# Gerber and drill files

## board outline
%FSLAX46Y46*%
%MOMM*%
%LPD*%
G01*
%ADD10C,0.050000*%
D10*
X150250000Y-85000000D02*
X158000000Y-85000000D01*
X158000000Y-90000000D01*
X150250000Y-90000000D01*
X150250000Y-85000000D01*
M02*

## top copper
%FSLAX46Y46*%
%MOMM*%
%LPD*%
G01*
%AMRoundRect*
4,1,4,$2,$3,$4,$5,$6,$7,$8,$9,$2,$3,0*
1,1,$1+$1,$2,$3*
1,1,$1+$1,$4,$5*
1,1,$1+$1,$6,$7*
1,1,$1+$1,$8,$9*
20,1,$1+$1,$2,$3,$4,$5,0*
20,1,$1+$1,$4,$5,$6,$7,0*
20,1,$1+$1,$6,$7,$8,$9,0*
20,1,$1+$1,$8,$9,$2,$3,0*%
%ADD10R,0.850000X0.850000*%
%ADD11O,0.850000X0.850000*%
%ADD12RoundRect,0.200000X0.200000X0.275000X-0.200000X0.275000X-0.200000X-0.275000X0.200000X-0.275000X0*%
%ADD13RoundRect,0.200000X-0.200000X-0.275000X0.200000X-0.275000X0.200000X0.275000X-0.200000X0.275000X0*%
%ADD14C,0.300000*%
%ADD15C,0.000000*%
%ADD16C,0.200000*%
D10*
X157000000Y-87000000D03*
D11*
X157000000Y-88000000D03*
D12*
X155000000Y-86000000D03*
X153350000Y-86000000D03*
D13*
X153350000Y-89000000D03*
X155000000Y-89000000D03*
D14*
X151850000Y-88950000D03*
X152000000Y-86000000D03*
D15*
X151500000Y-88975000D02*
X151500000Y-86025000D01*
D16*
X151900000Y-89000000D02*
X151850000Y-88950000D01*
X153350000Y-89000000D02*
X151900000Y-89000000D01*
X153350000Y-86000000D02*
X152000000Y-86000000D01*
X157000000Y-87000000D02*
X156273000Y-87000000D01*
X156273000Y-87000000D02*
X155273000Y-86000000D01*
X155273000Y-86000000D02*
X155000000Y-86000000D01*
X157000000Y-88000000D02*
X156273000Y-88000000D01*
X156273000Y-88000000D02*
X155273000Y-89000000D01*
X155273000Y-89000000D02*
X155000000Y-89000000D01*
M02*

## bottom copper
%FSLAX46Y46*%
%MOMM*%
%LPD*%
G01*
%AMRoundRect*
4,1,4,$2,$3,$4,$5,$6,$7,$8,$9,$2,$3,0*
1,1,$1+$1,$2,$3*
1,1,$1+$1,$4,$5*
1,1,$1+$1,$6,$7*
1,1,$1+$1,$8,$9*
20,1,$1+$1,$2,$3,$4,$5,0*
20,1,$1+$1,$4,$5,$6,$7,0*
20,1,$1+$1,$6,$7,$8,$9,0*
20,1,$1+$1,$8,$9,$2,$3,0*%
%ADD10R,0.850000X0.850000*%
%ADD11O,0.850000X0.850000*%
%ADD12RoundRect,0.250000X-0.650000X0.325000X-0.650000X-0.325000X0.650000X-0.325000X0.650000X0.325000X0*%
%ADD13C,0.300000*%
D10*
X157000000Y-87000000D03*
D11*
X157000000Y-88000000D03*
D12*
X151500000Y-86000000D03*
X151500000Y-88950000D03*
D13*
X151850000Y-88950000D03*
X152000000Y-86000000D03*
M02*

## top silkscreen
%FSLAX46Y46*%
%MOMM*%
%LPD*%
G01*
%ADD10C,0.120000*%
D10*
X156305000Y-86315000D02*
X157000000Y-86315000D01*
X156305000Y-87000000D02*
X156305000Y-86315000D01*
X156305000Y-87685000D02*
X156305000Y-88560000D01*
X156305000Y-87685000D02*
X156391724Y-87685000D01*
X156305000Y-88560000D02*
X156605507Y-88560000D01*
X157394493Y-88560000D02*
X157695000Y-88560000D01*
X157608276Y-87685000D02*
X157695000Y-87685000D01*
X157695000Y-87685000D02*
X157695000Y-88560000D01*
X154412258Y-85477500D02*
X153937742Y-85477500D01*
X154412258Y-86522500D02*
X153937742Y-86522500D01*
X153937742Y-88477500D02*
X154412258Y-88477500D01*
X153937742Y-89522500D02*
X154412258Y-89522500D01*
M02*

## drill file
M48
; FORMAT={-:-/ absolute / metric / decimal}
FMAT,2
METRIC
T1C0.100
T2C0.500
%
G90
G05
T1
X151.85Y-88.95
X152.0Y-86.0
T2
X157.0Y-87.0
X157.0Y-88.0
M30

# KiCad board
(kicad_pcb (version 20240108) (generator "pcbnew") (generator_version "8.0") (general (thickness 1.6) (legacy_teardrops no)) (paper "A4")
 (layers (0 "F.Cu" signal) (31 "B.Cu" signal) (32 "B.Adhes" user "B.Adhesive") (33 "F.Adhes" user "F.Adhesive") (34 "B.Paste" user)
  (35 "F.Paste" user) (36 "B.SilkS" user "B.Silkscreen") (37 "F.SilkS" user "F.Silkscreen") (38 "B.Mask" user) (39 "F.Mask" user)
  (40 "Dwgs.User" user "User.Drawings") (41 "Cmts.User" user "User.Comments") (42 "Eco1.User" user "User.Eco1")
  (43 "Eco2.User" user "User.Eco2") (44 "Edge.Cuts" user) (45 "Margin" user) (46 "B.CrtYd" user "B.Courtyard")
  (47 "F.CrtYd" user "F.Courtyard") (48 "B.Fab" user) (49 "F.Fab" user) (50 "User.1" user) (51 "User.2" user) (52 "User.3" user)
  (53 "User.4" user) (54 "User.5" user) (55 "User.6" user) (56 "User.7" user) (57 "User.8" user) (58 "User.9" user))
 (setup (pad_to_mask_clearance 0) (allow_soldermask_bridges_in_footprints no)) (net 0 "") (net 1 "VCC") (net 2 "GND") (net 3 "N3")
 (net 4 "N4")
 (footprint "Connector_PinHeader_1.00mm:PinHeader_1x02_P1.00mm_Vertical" (layer "F.Cu") (at 157 87)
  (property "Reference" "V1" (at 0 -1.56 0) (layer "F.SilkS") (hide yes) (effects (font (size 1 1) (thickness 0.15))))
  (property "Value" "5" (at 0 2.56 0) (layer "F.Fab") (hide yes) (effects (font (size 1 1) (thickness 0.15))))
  (fp_line (start -0.695 -0.685) (end 0 -0.685) (stroke (width 0.12) (type solid)) (layer "F.SilkS"))
  (fp_line (start -0.695 0) (end -0.695 -0.685) (stroke (width 0.12) (type solid)) (layer "F.SilkS"))
  (fp_line (start -0.695 0.685) (end -0.695 1.56) (stroke (width 0.12) (type solid)) (layer "F.SilkS"))
  (fp_line (start -0.695 0.685) (end -0.608276 0.685) (stroke (width 0.12) (type solid)) (layer "F.SilkS"))
  (fp_line (start -0.695 1.56) (end -0.394493 1.56) (stroke (width 0.12) (type solid)) (layer "F.SilkS"))
  (fp_line (start 0.394493 1.56) (end 0.695 1.56) (stroke (width 0.12) (type solid)) (layer "F.SilkS"))
  (fp_line (start 0.608276 0.685) (end 0.695 0.685) (stroke (width 0.12) (type solid)) (layer "F.SilkS"))
  (fp_line (start 0.695 0.685) (end 0.695 1.56) (stroke (width 0.12) (type solid)) (layer "F.SilkS"))
  (pad "1" thru_hole rect (at 0 0) (size 0.85 0.85) (drill 0.5) (layers "*.Cu" "*.Mask") (remove_unused_layers no) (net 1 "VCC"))
  (pad "2" thru_hole oval (at 0 1) (size 0.85 0.85) (drill 0.5) (layers "*.Cu" "*.Mask") (remove_unused_layers no) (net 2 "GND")))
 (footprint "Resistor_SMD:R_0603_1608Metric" (layer "F.Cu") (at 154.175 86 180)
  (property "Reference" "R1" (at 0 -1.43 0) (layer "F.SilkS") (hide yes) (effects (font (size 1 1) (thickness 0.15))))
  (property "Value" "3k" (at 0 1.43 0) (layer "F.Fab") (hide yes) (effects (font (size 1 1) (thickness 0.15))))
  (fp_line (start -0.237258 0.5225) (end 0.237258 0.5225) (stroke (width 0.12) (type solid)) (layer "F.SilkS"))
  (fp_line (start -0.237258 -0.5225) (end 0.237258 -0.5225) (stroke (width 0.12) (type solid)) (layer "F.SilkS"))
  (pad "1" smd roundrect (at -0.825 0 180) (size 0.8 0.95) (layers "F.Cu" "F.Paste" "F.Mask") (roundrect_rratio 0.25) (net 1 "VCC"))
  (pad "2" smd roundrect (at 0.825 0 180) (size 0.8 0.95) (layers "F.Cu" "F.Paste" "F.Mask") (roundrect_rratio 0.25) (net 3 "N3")))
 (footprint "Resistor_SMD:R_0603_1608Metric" (layer "F.Cu") (at 154.175 89)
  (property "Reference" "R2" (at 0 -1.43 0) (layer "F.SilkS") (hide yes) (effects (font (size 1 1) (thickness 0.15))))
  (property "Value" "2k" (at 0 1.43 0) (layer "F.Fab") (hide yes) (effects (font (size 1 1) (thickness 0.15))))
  (fp_line (start -0.237258 -0.5225) (end 0.237258 -0.5225) (stroke (width 0.12) (type solid)) (layer "F.SilkS"))
  (fp_line (start -0.237258 0.5225) (end 0.237258 0.5225) (stroke (width 0.12) (type solid)) (layer "F.SilkS"))
  (pad "1" smd roundrect (at -0.825 0) (size 0.8 0.95) (layers "F.Cu" "F.Paste" "F.Mask") (roundrect_rratio 0.25) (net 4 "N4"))
  (pad "2" smd roundrect (at 0.825 0) (size 0.8 0.95) (layers "F.Cu" "F.Paste" "F.Mask") (roundrect_rratio 0.25) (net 2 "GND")))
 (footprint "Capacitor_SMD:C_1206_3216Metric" (layer "B.Cu") (at 151.5 87.475 -90)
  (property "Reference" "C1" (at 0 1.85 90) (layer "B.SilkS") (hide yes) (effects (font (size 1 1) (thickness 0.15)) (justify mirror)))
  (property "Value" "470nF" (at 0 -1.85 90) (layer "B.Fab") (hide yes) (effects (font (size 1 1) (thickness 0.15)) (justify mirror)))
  (pad "1" smd roundrect (at -1.475 0 270) (size 1.15 1.8) (layers "B.Cu" "B.Paste" "B.Mask") (roundrect_rratio 0.217391) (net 3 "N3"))
  (pad "2" smd roundrect (at 1.475 0 270) (size 1.15 1.8) (layers "B.Cu" "B.Paste" "B.Mask") (roundrect_rratio 0.217391) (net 4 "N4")))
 (gr_rect (start 150.25 85) (end 158 90) (stroke (width 0.05) (type default)) (fill none) (layer "Edge.Cuts"))
 (segment (start 151.5 88.975) (end 151.5 86.025) (width 0) (layer "F.Cu") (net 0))
 (segment (start 151.9 89) (end 151.85 88.95) (width 0.2) (layer "F.Cu") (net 4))
 (segment (start 153.35 89) (end 151.9 89) (width 0.2) (layer "F.Cu") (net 4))
 (via micro (at 151.85 88.95) (size 0.3) (drill 0.1) (layers "F.Cu" "B.Cu") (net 4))
 (segment (start 153.35 86) (end 152 86) (width 0.2) (layer "F.Cu") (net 3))
 (via micro (at 152 86) (size 0.3) (drill 0.1) (layers "F.Cu" "B.Cu") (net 3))
 (segment (start 157 87) (end 156.273 87) (width 0.2) (layer "F.Cu") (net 1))
 (segment (start 156.273 87) (end 155.273 86) (width 0.2) (layer "F.Cu") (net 1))
 (segment (start 155.273 86) (end 155 86) (width 0.2) (layer "F.Cu") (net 1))
 (segment (start 157 88) (end 156.273 88) (width 0.2) (layer "F.Cu") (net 2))
 (segment (start 156.273 88) (end 155.273 89) (width 0.2) (layer "F.Cu") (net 2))
 (segment (start 155.273 89) (end 155 89) (width 0.2) (layer "F.Cu") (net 2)))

